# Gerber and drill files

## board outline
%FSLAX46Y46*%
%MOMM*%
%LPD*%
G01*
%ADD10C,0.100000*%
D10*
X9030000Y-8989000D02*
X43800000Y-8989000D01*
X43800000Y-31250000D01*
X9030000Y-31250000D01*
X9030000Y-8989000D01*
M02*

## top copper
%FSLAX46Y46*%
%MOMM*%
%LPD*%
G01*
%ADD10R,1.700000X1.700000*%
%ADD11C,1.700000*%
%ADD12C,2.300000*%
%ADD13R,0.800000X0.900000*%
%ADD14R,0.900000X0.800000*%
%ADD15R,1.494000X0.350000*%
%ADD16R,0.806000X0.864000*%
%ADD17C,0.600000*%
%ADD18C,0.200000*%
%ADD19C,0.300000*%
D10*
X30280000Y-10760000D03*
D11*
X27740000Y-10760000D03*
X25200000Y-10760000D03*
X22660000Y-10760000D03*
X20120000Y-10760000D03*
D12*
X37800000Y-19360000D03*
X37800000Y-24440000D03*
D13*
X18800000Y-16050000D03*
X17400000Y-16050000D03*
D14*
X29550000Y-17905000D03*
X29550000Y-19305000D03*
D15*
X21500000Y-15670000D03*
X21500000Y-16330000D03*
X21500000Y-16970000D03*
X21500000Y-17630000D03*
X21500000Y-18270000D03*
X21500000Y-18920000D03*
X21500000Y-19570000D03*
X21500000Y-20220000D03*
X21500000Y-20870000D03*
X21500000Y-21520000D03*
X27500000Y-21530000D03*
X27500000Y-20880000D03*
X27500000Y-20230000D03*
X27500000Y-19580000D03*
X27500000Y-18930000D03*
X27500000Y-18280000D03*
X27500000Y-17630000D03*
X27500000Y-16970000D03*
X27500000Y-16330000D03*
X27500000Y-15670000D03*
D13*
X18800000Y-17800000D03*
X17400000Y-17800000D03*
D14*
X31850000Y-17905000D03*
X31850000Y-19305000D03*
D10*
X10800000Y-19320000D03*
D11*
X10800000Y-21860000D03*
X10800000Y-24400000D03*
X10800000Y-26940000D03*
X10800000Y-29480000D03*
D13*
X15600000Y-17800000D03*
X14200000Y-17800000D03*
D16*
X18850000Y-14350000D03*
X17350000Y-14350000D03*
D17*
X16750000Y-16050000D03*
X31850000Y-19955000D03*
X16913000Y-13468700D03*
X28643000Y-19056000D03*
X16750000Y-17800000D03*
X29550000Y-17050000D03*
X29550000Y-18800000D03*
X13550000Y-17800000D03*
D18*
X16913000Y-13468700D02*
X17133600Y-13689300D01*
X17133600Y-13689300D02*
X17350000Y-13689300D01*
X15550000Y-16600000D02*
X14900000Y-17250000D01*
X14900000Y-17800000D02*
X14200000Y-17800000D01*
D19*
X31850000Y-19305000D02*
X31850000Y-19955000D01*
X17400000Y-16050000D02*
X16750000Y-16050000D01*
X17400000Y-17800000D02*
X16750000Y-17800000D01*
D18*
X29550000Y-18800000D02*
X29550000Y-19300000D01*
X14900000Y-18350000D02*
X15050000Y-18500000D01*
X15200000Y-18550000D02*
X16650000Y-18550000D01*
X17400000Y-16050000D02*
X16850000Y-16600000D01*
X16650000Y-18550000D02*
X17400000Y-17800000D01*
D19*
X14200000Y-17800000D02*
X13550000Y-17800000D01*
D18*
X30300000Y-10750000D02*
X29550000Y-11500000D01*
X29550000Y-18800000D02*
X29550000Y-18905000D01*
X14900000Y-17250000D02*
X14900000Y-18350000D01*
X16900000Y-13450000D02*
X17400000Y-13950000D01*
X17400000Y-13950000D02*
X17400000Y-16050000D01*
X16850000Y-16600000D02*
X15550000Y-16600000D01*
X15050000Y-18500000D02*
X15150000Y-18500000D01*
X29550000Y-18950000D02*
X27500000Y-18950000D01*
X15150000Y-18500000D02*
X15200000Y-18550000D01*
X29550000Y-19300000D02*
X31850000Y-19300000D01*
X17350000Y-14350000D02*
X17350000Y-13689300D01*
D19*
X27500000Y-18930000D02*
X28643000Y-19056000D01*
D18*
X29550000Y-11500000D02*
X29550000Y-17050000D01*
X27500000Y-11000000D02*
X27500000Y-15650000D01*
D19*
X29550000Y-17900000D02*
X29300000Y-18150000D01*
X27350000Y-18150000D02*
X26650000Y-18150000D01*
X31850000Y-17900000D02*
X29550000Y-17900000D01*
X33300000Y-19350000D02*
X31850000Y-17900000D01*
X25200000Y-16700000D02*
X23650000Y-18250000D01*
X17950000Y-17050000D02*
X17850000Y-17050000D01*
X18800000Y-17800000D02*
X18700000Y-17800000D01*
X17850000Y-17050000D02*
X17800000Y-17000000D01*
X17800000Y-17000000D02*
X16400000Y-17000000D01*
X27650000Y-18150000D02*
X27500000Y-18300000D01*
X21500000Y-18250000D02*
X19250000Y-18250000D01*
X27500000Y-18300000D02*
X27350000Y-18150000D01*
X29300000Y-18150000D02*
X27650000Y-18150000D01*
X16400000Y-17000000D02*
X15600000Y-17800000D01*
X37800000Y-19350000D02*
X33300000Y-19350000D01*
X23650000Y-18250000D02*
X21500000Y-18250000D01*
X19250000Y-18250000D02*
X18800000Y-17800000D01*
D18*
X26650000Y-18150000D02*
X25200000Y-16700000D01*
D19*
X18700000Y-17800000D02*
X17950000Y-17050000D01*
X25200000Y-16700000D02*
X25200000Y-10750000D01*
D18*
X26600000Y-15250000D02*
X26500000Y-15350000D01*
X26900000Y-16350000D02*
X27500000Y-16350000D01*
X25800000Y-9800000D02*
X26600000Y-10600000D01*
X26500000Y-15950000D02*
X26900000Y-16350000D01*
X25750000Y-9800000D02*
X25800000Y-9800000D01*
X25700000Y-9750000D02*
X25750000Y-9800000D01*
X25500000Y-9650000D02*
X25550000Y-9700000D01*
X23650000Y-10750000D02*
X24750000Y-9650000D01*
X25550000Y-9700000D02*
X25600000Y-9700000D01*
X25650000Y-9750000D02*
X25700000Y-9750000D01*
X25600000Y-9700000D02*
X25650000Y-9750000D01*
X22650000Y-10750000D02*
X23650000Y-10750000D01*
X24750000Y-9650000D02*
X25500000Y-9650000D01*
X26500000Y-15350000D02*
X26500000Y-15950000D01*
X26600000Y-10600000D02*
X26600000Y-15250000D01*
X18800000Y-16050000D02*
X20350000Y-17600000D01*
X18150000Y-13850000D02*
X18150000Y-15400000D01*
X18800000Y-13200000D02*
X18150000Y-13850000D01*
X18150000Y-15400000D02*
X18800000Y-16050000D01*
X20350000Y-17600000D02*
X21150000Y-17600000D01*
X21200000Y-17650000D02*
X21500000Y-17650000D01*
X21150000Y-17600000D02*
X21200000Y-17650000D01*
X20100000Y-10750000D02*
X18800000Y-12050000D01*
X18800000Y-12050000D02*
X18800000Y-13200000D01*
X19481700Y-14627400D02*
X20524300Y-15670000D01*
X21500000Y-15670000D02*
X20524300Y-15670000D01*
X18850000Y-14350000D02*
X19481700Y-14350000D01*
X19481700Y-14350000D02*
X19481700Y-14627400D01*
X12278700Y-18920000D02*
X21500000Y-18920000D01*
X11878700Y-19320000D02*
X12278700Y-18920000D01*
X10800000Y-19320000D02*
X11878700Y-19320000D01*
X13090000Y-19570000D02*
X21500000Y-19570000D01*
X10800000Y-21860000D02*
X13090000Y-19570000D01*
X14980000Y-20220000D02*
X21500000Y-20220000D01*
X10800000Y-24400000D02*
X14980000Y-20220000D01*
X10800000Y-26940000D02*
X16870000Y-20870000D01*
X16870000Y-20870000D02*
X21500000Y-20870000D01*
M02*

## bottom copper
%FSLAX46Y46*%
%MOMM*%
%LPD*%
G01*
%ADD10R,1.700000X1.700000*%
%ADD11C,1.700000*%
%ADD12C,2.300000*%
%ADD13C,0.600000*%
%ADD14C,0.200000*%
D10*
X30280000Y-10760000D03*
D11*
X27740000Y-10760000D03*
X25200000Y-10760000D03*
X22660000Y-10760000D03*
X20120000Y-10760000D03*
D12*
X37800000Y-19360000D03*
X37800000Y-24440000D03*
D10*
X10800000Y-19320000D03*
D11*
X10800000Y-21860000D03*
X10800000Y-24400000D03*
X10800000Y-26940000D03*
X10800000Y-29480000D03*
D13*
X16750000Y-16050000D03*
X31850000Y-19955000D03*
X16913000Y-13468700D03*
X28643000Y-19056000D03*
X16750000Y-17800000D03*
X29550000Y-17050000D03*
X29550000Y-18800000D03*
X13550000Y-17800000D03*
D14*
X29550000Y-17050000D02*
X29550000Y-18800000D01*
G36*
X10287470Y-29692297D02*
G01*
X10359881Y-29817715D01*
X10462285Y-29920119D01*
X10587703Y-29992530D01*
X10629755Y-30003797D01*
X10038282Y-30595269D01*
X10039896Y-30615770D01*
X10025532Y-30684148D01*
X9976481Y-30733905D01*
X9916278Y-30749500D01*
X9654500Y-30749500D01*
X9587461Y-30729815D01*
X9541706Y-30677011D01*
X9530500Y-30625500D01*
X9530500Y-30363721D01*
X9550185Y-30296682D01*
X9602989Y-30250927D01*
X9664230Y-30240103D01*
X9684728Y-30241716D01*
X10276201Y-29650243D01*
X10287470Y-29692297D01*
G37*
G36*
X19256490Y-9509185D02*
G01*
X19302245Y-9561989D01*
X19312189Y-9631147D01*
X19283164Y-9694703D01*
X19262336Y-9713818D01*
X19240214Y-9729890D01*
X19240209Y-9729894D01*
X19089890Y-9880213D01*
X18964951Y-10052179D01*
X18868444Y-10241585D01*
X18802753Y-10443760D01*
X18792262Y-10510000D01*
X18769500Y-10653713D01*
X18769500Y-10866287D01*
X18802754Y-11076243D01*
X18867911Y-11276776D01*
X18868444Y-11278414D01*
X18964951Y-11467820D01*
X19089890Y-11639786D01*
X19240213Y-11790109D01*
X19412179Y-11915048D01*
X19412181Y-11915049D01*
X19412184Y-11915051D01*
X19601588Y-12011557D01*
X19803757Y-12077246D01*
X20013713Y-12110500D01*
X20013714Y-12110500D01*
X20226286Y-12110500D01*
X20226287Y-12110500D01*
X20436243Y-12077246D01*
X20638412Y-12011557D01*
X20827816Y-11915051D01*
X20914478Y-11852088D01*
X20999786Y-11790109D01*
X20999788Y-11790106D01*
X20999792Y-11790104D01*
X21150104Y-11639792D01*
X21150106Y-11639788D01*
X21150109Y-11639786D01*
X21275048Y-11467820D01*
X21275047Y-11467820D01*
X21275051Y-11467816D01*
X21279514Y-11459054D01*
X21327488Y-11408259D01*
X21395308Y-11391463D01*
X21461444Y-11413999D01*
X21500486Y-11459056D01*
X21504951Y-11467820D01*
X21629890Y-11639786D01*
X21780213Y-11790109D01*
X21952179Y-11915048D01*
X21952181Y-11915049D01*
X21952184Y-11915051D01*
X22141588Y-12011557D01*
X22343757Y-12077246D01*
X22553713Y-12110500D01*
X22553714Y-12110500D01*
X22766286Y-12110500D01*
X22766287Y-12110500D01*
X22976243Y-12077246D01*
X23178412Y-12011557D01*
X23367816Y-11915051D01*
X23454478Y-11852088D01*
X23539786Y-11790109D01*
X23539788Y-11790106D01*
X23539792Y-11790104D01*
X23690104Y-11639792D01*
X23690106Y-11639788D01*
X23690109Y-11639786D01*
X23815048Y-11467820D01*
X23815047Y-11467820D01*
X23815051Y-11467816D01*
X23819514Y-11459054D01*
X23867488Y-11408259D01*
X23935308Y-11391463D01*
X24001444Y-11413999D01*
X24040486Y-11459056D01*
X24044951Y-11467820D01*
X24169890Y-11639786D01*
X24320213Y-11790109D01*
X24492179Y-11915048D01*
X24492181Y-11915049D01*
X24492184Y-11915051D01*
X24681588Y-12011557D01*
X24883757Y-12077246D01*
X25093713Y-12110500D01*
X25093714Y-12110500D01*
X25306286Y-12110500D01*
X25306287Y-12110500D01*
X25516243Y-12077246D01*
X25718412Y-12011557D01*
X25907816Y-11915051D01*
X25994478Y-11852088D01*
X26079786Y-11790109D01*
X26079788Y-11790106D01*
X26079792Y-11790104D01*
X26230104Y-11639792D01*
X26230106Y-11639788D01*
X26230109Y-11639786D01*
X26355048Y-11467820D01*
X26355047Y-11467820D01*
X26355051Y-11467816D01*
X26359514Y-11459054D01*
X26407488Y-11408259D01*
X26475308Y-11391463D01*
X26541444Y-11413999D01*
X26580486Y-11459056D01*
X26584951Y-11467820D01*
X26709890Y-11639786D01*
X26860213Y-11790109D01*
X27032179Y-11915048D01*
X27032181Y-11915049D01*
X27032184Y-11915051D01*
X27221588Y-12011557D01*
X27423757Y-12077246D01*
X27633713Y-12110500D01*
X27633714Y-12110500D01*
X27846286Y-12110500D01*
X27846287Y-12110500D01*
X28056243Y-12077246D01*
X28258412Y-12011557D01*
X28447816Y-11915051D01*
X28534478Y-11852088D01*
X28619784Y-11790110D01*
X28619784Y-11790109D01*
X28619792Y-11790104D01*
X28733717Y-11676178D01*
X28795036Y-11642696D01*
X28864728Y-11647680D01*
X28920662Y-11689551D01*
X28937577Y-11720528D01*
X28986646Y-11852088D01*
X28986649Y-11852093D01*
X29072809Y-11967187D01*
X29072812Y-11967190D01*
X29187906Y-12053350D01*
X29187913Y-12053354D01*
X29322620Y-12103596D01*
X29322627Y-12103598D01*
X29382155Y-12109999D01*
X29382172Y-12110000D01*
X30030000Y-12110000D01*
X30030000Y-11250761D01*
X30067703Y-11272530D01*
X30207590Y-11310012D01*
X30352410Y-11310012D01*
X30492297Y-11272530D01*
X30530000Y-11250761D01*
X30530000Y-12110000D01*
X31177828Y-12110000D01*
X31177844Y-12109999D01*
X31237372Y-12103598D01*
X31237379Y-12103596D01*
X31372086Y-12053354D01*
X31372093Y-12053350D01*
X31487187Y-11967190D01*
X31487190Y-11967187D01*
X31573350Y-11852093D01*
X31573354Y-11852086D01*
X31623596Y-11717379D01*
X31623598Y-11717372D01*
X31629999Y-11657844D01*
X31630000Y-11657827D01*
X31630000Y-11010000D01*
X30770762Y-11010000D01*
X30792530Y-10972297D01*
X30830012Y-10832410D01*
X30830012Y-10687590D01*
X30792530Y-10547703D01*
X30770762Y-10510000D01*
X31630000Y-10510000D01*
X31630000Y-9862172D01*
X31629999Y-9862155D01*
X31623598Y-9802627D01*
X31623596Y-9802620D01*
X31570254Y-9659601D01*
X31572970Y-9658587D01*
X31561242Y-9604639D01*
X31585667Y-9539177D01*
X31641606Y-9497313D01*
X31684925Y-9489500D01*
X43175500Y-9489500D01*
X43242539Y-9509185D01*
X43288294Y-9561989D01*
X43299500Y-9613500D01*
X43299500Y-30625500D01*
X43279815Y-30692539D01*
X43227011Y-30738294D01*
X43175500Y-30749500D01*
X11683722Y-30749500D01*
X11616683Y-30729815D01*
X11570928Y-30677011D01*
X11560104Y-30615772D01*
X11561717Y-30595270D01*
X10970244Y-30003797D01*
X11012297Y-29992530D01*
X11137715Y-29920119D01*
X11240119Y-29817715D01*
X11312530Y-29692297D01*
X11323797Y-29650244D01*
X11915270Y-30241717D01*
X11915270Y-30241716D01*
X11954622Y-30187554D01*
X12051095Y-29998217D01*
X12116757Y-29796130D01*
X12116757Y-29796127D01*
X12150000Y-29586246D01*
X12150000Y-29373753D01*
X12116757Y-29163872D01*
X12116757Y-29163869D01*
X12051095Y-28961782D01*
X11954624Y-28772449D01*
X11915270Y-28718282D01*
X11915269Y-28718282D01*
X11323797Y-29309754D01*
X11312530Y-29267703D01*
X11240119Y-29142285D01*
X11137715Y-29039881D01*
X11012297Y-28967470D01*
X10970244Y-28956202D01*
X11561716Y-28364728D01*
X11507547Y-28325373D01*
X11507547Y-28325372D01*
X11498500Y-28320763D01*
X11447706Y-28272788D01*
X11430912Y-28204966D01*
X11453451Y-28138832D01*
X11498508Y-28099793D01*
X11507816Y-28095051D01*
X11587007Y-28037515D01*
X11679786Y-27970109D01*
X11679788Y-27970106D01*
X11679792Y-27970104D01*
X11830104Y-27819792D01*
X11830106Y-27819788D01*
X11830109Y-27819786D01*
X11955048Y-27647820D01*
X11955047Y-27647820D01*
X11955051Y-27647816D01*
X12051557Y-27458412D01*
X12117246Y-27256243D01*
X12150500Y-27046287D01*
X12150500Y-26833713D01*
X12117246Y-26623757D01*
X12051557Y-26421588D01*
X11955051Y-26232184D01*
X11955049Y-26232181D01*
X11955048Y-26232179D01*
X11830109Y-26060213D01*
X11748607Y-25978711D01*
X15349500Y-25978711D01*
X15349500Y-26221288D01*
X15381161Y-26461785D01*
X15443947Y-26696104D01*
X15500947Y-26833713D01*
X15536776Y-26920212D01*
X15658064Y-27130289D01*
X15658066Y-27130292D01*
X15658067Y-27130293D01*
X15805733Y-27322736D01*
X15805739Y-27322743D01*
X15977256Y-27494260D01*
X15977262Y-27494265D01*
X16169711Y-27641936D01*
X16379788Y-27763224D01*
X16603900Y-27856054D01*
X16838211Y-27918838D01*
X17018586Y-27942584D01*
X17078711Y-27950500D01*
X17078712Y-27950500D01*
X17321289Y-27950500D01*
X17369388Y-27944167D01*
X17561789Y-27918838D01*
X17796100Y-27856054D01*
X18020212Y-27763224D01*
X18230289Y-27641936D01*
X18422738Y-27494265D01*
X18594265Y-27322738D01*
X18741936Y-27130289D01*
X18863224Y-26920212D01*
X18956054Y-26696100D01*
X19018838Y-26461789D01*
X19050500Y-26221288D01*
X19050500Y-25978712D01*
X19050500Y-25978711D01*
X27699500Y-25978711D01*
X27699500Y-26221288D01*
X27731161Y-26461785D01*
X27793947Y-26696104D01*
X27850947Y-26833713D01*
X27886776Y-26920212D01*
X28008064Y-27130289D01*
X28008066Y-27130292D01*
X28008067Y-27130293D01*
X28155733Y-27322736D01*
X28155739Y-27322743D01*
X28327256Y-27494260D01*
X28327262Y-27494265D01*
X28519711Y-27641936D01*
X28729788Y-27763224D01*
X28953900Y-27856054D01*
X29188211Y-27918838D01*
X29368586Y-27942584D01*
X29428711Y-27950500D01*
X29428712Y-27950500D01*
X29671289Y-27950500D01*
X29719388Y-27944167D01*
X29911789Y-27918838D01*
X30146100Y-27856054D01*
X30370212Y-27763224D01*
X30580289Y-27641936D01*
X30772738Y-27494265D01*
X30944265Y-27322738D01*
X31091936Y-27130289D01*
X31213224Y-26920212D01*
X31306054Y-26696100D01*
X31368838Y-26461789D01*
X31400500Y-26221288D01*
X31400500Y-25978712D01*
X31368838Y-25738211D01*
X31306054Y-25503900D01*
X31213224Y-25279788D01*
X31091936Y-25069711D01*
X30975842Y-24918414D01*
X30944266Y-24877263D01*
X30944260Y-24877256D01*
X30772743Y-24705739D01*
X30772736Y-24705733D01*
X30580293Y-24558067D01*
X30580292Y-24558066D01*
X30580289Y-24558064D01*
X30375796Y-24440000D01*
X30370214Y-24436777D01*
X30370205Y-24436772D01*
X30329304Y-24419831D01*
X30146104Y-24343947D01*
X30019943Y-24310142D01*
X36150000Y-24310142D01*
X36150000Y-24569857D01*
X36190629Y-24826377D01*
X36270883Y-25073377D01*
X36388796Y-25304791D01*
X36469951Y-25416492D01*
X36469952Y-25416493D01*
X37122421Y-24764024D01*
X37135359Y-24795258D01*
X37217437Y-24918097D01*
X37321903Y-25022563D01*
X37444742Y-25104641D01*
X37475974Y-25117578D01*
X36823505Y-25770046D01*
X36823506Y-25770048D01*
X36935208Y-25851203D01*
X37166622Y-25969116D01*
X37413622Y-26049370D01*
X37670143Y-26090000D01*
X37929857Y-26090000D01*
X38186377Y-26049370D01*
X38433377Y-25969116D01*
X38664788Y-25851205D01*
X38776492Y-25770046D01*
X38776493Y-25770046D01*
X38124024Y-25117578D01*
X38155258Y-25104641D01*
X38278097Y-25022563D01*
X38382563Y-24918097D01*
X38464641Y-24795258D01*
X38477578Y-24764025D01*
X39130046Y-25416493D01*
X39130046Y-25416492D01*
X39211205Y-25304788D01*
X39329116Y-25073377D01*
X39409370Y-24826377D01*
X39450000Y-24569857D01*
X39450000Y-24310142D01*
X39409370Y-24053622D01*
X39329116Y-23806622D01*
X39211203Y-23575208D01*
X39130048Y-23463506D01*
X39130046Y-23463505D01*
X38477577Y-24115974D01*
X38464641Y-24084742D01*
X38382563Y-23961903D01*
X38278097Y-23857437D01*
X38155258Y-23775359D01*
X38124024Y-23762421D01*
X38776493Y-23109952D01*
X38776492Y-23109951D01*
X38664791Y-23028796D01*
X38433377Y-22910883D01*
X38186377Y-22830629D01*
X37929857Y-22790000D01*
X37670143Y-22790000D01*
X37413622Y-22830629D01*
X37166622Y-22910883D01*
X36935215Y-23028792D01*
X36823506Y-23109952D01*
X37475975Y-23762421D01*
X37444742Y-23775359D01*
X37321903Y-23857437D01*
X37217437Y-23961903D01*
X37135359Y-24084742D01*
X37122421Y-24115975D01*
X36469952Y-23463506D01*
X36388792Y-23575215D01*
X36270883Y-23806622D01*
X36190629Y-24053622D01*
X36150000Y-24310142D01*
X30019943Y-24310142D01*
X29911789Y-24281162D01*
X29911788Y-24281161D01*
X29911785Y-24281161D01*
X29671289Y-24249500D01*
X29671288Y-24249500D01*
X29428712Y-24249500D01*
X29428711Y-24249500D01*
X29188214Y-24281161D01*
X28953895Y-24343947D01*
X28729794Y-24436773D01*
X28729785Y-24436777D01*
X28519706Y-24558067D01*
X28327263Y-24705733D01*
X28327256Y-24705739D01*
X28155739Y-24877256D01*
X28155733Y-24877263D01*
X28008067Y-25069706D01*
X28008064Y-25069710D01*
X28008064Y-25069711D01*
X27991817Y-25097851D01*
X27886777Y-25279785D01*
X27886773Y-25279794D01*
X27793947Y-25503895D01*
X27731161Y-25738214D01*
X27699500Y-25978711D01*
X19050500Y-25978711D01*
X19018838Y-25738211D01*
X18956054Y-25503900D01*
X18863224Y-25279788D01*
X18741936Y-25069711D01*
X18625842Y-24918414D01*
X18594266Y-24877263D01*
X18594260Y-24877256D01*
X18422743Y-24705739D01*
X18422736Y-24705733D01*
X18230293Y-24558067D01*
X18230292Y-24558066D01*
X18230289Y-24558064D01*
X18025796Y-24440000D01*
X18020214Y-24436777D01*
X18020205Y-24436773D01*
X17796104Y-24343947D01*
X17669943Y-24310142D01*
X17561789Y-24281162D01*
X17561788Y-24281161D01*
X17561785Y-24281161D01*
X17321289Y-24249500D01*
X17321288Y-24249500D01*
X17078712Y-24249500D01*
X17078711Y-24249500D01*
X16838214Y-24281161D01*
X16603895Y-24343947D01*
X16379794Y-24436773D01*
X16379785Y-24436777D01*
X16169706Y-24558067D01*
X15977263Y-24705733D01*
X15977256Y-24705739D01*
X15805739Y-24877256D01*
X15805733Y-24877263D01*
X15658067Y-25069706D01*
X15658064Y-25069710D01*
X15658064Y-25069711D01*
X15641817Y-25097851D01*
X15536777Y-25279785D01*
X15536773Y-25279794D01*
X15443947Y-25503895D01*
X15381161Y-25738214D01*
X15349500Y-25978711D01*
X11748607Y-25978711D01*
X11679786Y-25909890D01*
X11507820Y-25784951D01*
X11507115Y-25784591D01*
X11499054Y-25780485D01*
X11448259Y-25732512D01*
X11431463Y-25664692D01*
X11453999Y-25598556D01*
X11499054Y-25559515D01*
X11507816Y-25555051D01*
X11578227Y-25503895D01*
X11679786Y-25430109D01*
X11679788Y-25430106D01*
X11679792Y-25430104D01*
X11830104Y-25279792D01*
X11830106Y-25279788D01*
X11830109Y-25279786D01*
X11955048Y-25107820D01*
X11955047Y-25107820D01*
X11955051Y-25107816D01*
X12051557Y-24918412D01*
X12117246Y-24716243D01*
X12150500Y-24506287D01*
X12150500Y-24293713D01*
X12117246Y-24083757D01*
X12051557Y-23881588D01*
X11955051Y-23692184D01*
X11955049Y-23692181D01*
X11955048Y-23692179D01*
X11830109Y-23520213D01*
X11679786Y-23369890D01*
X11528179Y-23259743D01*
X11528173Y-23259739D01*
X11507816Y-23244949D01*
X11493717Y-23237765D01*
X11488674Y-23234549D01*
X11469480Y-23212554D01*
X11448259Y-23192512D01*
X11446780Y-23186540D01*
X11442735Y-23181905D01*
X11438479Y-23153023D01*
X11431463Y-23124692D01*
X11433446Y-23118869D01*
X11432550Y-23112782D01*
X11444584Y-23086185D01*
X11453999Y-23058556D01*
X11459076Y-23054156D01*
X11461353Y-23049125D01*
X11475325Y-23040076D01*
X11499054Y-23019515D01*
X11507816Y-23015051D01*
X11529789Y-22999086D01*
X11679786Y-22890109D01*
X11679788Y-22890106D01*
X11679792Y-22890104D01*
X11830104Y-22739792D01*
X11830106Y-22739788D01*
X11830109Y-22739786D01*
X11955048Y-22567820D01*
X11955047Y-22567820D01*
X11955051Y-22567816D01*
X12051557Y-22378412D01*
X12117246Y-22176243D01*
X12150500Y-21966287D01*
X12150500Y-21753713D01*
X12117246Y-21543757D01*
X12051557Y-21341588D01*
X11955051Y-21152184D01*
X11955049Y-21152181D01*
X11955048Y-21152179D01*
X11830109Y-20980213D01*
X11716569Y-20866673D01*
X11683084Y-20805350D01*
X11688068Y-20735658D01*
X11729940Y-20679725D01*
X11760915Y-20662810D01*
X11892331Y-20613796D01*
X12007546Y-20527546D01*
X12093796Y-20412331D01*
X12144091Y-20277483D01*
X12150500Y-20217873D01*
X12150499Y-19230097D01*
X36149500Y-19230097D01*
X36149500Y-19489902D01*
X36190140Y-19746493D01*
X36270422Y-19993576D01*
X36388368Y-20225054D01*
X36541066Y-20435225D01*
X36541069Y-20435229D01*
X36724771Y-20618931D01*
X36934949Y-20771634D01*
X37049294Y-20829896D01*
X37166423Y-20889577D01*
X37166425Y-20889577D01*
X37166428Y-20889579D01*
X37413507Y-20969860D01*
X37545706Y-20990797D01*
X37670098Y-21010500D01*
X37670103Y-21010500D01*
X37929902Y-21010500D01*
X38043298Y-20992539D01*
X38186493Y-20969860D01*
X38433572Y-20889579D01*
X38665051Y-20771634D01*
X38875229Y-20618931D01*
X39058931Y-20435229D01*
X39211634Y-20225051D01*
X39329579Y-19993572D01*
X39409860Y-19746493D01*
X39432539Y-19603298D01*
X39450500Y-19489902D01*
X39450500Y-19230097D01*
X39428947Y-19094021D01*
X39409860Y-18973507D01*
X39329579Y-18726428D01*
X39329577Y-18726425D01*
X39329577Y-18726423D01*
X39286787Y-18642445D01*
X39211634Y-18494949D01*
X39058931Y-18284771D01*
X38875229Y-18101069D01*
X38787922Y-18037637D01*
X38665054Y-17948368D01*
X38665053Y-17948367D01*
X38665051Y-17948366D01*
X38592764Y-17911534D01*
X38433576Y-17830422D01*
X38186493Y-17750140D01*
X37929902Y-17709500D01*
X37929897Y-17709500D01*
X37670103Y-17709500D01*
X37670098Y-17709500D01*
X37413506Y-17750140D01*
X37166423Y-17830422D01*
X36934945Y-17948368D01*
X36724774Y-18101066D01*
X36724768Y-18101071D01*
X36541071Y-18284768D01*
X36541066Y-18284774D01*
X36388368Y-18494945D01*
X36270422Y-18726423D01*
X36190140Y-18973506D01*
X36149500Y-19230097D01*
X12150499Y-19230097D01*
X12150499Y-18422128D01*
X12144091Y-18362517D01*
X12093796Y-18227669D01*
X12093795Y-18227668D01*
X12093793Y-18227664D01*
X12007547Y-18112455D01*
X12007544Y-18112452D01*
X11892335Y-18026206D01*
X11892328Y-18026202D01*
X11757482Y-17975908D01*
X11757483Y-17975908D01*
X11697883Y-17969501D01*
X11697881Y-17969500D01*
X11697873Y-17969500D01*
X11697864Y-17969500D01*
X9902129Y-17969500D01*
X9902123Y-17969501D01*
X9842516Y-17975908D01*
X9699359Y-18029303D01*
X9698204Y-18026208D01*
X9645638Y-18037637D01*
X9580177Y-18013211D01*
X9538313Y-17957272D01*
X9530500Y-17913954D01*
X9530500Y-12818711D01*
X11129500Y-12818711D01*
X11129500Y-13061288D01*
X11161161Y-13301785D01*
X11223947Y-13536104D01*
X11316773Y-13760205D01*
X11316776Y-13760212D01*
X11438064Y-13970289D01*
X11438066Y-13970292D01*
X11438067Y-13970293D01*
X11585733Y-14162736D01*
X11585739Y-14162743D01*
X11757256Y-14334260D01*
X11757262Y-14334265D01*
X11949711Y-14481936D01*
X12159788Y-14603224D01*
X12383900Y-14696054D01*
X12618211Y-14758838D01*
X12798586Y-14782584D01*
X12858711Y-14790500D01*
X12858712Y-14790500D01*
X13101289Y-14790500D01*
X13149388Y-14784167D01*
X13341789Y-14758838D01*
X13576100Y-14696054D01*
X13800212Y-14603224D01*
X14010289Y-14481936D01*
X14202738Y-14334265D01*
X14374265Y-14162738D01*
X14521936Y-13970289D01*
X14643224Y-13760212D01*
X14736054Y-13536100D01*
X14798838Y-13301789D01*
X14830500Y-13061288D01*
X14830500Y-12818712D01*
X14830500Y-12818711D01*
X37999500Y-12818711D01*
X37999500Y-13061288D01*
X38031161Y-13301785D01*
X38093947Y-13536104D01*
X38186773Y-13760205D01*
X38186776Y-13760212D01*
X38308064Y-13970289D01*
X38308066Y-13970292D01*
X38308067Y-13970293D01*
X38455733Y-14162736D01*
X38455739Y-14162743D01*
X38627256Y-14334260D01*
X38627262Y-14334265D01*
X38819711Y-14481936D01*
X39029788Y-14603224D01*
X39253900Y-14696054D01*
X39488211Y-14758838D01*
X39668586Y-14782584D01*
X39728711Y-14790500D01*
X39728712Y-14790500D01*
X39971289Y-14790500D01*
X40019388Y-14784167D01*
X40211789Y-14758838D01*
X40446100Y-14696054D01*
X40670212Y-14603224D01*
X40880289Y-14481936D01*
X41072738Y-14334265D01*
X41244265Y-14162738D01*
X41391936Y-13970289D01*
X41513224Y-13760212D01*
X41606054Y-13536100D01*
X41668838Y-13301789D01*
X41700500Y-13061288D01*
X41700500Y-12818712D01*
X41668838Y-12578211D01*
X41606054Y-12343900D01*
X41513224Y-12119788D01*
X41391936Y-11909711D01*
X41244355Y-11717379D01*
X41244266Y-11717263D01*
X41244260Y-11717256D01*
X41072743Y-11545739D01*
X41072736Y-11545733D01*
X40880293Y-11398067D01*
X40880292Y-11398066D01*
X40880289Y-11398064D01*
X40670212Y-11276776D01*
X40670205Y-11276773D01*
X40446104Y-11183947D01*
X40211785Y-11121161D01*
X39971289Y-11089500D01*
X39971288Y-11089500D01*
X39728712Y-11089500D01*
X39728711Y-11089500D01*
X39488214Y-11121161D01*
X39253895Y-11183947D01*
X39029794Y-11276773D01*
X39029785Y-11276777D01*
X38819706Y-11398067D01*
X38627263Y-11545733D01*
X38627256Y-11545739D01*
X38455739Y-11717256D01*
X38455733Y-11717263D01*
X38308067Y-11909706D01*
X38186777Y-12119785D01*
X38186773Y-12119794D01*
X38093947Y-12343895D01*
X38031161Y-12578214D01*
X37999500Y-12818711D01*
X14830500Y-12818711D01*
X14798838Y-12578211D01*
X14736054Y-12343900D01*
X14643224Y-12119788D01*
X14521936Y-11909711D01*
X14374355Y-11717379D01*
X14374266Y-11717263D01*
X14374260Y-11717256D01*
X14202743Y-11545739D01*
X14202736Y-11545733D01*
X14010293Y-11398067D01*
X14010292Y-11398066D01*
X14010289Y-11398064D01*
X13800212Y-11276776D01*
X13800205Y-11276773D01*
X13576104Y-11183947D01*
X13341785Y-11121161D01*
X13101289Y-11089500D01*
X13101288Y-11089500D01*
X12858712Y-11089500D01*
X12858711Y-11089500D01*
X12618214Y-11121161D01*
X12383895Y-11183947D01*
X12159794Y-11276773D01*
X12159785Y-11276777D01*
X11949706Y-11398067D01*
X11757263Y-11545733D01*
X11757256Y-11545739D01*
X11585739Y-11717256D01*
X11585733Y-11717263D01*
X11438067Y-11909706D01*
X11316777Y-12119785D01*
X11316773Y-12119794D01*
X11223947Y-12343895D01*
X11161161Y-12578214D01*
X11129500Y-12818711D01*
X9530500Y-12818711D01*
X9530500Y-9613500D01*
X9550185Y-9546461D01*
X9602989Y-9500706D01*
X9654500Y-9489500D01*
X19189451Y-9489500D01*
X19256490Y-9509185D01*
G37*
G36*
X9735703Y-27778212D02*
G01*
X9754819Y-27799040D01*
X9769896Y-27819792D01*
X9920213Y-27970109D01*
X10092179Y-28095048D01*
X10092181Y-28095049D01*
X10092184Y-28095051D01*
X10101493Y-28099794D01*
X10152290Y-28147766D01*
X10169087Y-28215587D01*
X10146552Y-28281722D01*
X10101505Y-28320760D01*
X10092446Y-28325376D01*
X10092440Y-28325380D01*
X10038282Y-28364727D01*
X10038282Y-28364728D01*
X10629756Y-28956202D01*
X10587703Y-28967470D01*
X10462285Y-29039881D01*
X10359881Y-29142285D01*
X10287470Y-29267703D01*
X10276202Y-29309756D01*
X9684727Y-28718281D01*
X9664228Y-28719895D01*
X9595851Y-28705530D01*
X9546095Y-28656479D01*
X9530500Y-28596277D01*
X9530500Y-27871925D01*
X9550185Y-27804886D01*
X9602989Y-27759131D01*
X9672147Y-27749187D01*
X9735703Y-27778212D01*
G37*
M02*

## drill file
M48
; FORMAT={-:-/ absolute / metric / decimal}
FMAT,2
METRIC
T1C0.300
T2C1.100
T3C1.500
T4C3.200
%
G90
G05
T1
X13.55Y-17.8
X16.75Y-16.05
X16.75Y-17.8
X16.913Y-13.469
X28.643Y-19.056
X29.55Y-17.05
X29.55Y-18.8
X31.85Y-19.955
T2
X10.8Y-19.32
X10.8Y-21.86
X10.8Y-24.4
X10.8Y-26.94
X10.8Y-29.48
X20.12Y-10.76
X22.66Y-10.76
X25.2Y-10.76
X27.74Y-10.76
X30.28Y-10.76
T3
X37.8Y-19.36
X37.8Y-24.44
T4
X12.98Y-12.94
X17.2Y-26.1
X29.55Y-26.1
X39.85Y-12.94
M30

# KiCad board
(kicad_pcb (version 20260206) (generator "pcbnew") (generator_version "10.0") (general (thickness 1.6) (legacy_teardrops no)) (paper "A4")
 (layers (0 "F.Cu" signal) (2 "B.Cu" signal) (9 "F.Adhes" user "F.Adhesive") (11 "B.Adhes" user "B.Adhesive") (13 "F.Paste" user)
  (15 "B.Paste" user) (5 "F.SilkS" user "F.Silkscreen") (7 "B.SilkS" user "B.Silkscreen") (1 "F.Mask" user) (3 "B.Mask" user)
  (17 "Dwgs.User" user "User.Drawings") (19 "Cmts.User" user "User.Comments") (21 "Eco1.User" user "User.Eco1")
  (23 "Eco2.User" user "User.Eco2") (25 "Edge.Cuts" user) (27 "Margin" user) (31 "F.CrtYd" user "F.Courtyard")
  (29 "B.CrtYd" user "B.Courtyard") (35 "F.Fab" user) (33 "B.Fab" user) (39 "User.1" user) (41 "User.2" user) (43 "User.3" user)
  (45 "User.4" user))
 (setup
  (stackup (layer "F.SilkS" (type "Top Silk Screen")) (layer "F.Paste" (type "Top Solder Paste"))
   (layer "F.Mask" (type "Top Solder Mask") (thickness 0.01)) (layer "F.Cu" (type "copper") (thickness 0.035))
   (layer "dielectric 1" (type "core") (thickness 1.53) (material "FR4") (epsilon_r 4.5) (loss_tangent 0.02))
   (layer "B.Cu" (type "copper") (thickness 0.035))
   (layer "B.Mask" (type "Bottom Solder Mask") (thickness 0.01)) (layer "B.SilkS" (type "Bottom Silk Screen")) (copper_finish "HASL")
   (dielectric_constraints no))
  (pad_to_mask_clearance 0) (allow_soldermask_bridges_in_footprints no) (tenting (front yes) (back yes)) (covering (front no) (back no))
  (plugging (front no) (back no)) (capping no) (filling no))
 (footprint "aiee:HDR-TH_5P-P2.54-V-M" (layer "F.Cu") (at 25.2 10.76 180)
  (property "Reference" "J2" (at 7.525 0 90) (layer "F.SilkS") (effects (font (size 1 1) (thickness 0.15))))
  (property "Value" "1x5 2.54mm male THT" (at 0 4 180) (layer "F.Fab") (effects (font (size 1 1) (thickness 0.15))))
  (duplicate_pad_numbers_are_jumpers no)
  (pad "1" thru_hole rect (at -5.08 0 180) (size 1.7 1.7) (drill 1.100024) (layers "*.Cu" "*.Mask") (remove_unused_layers no) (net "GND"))
  (pad "2" thru_hole circle (at -2.54 0 180) (size 1.7 1.7) (drill 1.100024) (layers "*.Cu" "*.Mask") (remove_unused_layers no)
   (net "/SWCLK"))
  (pad "3" thru_hole circle (at 0 0 180) (size 1.7 1.7) (drill 1.100024) (layers "*.Cu" "*.Mask") (remove_unused_layers no) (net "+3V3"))
  (pad "4" thru_hole circle (at 2.54 0 180) (size 1.7 1.7) (drill 1.100024) (layers "*.Cu" "*.Mask") (remove_unused_layers no)
   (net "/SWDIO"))
  (pad "5" thru_hole circle (at 5.08 0 180) (size 1.7 1.7) (drill 1.100024) (layers "*.Cu" "*.Mask") (remove_unused_layers no) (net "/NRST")))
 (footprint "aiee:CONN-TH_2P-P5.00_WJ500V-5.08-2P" (layer "F.Cu") (at 37.8 21.9 -90)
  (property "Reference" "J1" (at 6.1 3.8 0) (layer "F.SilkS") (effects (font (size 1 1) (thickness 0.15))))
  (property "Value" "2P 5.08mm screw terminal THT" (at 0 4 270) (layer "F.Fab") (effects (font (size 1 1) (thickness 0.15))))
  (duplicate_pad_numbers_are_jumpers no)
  (pad "1" thru_hole circle (at -2.54 0 90) (size 2.3 2.3) (drill 1.5) (layers "*.Cu" "*.Mask") (remove_unused_layers no) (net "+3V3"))
  (pad "2" thru_hole circle (at 2.54 0 90) (size 2.3 2.3) (drill 1.5) (layers "*.Cu" "*.Mask") (remove_unused_layers no) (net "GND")))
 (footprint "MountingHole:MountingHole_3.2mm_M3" (layer "F.Cu") (at 29.55 26.1)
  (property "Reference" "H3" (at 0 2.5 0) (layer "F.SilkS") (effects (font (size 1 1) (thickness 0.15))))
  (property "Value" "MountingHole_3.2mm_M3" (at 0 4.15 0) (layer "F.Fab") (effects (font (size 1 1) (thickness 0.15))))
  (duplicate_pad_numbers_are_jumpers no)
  (pad "" np_thru_hole circle (at 0 0) (size 3.2 3.2) (drill 3.2) (layers "*.Cu" "*.Mask")))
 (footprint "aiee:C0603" (layer "F.Cu") (at 18.1 16.05 180)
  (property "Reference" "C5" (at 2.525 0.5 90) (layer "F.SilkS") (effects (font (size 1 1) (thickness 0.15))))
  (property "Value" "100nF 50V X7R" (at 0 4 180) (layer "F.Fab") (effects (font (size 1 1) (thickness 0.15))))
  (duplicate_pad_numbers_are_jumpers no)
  (pad "1" smd rect (at -0.7 0 180) (size 0.8 0.9) (layers "F.Cu" "F.Mask" "F.Paste") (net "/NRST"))
  (pad "2" smd rect (at 0.7 0 180) (size 0.8 0.9) (layers "F.Cu" "F.Mask" "F.Paste") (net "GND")))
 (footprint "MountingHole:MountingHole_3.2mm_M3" (layer "F.Cu") (at 17.2 26.1)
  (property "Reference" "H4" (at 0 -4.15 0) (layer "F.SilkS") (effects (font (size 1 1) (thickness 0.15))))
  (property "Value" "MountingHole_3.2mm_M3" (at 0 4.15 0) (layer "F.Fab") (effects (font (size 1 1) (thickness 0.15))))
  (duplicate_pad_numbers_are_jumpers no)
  (pad "" np_thru_hole circle (at 0 0) (size 3.2 3.2) (drill 3.2) (layers "*.Cu" "*.Mask")))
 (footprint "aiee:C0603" (layer "F.Cu") (at 29.55 18.605 -90)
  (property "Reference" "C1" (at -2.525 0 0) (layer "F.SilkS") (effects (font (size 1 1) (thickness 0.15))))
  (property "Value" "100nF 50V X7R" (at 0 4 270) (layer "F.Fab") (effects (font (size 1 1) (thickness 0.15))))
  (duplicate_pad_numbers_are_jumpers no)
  (pad "1" smd rect (at -0.7 0 270) (size 0.8 0.9) (layers "F.Cu" "F.Mask" "F.Paste") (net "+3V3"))
  (pad "2" smd rect (at 0.7 0 270) (size 0.8 0.9) (layers "F.Cu" "F.Mask" "F.Paste") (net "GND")))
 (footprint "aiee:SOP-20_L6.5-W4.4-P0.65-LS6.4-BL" (layer "F.Cu") (at 24.5 18.6 -90)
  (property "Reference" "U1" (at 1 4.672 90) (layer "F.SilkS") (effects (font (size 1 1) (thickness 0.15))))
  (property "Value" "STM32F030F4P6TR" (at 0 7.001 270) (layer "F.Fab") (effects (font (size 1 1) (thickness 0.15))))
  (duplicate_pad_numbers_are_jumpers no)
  (pad "1" smd rect (at -2.93 3 270) (size 0.35 1.494) (layers "F.Cu" "F.Mask" "F.Paste") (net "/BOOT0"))
  (pad "2" smd rect (at -2.27 3 270) (size 0.35 1.494) (layers "F.Cu" "F.Mask" "F.Paste") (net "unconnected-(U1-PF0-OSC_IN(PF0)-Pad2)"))
  (pad "3" smd rect (at -1.63 3 270) (size 0.35 1.494) (layers "F.Cu" "F.Mask" "F.Paste") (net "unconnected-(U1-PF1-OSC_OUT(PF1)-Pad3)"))
  (pad "4" smd rect (at -0.97 3 270) (size 0.35 1.494) (layers "F.Cu" "F.Mask" "F.Paste") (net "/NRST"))
  (pad "5" smd rect (at -0.33 3 270) (size 0.35 1.494) (layers "F.Cu" "F.Mask" "F.Paste") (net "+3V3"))
  (pad "6" smd rect (at 0.32 3 270) (size 0.35 1.494) (layers "F.Cu" "F.Mask" "F.Paste") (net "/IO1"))
  (pad "7" smd rect (at 0.97 3 270) (size 0.35 1.494) (layers "F.Cu" "F.Mask" "F.Paste") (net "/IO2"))
  (pad "8" smd rect (at 1.62 3 270) (size 0.35 1.494) (layers "F.Cu" "F.Mask" "F.Paste") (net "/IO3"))
  (pad "9" smd rect (at 2.27 3 270) (size 0.35 1.494) (layers "F.Cu" "F.Mask" "F.Paste") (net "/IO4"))
  (pad "10" smd rect (at 2.92 3 270) (size 0.35 1.494) (layers "F.Cu" "F.Mask" "F.Paste") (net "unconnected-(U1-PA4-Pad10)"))
  (pad "11" smd rect (at 2.93 -3 270) (size 0.35 1.494) (layers "F.Cu" "F.Mask" "F.Paste") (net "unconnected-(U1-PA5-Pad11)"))
  (pad "12" smd rect (at 2.28 -3 270) (size 0.35 1.494) (layers "F.Cu" "F.Mask" "F.Paste") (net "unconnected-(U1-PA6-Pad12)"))
  (pad "13" smd rect (at 1.63 -3 270) (size 0.35 1.494) (layers "F.Cu" "F.Mask" "F.Paste") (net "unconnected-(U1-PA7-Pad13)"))
  (pad "14" smd rect (at 0.98 -3 270) (size 0.35 1.494) (layers "F.Cu" "F.Mask" "F.Paste") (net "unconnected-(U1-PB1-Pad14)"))
  (pad "15" smd rect (at 0.33 -3 270) (size 0.35 1.494) (layers "F.Cu" "F.Mask" "F.Paste") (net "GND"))
  (pad "16" smd rect (at -0.32 -3 270) (size 0.35 1.494) (layers "F.Cu" "F.Mask" "F.Paste") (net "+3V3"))
  (pad "17" smd rect (at -0.97 -3 270) (size 0.35 1.494) (layers "F.Cu" "F.Mask" "F.Paste") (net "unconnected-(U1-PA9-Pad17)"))
  (pad "18" smd rect (at -1.63 -3 270) (size 0.35 1.494) (layers "F.Cu" "F.Mask" "F.Paste") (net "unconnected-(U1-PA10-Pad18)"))
  (pad "19" smd rect (at -2.27 -3 270) (size 0.35 1.494) (layers "F.Cu" "F.Mask" "F.Paste") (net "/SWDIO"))
  (pad "20" smd rect (at -2.93 -3 270) (size 0.35 1.494) (layers "F.Cu" "F.Mask" "F.Paste") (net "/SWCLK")))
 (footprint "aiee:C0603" (layer "F.Cu") (at 18.1 17.8 180)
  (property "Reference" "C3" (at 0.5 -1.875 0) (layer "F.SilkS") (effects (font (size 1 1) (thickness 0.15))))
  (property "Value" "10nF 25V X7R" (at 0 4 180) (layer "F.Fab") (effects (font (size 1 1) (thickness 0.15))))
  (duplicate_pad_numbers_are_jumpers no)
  (pad "1" smd rect (at -0.7 0 180) (size 0.8 0.9) (layers "F.Cu" "F.Mask" "F.Paste") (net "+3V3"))
  (pad "2" smd rect (at 0.7 0 180) (size 0.8 0.9) (layers "F.Cu" "F.Mask" "F.Paste") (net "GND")))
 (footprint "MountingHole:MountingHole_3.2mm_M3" (layer "F.Cu") (at 12.98 12.94)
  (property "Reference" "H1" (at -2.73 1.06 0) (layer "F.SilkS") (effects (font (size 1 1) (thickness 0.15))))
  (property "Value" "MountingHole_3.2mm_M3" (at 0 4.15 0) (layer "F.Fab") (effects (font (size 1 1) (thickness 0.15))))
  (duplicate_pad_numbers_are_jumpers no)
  (pad "" np_thru_hole circle (at 0 0) (size 3.2 3.2) (drill 3.2) (layers "*.Cu" "*.Mask")))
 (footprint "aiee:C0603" (layer "F.Cu") (at 31.85 18.605 -90)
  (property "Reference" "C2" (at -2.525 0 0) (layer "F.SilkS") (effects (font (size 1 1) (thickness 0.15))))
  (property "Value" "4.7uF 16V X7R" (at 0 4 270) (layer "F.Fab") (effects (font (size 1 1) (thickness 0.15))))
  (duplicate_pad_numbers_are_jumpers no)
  (pad "1" smd rect (at -0.7 0 270) (size 0.8 0.9) (layers "F.Cu" "F.Mask" "F.Paste") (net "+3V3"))
  (pad "2" smd rect (at 0.7 0 270) (size 0.8 0.9) (layers "F.Cu" "F.Mask" "F.Paste") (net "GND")))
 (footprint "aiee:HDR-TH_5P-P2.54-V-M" (layer "F.Cu") (at 10.8 24.4 -90)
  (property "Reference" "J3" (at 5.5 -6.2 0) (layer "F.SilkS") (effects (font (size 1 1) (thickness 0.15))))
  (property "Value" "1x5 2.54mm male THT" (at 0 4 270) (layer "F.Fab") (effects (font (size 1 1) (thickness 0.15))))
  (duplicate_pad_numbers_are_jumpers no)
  (pad "1" thru_hole rect (at -5.08 0 270) (size 1.7 1.7) (drill 1.100024) (layers "*.Cu" "*.Mask") (remove_unused_layers no) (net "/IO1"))
  (pad "2" thru_hole circle (at -2.54 0 270) (size 1.7 1.7) (drill 1.100024) (layers "*.Cu" "*.Mask") (remove_unused_layers no) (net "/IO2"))
  (pad "3" thru_hole circle (at 0 0 270) (size 1.7 1.7) (drill 1.100024) (layers "*.Cu" "*.Mask") (remove_unused_layers no) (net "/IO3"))
  (pad "4" thru_hole circle (at 2.54 0 270) (size 1.7 1.7) (drill 1.100024) (layers "*.Cu" "*.Mask") (remove_unused_layers no) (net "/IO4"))
  (pad "5" thru_hole circle (at 5.08 0 270) (size 1.7 1.7) (drill 1.100024) (layers "*.Cu" "*.Mask") (remove_unused_layers no) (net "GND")))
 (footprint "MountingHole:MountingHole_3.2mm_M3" (layer "F.Cu") (at 39.85 12.94)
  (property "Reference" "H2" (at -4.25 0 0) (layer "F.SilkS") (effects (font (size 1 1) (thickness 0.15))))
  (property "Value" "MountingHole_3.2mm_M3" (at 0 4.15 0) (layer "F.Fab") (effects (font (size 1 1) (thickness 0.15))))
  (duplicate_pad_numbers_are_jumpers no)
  (pad "" np_thru_hole circle (at 0 0) (size 3.2 3.2) (drill 3.2) (layers "*.Cu" "*.Mask")))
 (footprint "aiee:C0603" (layer "F.Cu") (at 14.9 17.8 180)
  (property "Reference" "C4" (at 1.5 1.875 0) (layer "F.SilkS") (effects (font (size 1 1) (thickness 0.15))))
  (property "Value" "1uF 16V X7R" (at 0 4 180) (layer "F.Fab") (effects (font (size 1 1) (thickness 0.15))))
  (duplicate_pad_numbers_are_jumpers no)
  (pad "1" smd rect (at -0.7 0 180) (size 0.8 0.9) (layers "F.Cu" "F.Mask" "F.Paste") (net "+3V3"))
  (pad "2" smd rect (at 0.7 0 180) (size 0.8 0.9) (layers "F.Cu" "F.Mask" "F.Paste") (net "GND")))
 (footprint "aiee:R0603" (layer "F.Cu") (at 18.1 14.35 180)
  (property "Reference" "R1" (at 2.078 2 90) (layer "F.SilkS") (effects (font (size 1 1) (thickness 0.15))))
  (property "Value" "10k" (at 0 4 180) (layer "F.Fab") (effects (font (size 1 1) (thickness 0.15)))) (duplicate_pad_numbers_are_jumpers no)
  (pad "1" smd rect (at -0.75 0 180) (size 0.806 0.864) (layers "F.Cu" "F.Mask" "F.Paste") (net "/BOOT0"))
  (pad "2" smd rect (at 0.75 0 180) (size 0.806 0.864) (layers "F.Cu" "F.Mask" "F.Paste") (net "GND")))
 (gr_rect (start 9.03 8.989) (end 43.8 31.25) (stroke (width 0.1) (type default)) (fill no) (layer "Edge.Cuts"))
 (segment (start 16.913 13.4687) (end 17.1336 13.6893) (width 0.2) (layer "F.Cu") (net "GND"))
 (segment (start 17.1336 13.6893) (end 17.35 13.6893) (width 0.2) (layer "F.Cu") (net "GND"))
 (segment (start 15.55 16.6) (end 14.9 17.25) (width 0.2) (layer "F.Cu") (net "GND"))
 (segment (start 14.9 17.8) (end 14.2 17.8) (width 0.2) (layer "F.Cu") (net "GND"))
 (segment (start 31.85 19.305) (end 31.85 19.955) (width 0.3) (layer "F.Cu") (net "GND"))
 (segment (start 17.4 16.05) (end 16.75 16.05) (width 0.3) (layer "F.Cu") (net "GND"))
 (segment (start 17.4 17.8) (end 16.75 17.8) (width 0.3) (layer "F.Cu") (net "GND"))
 (segment (start 29.55 18.8) (end 29.55 19.3) (width 0.2) (layer "F.Cu") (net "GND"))
 (segment (start 14.9 18.35) (end 15.05 18.5) (width 0.2) (layer "F.Cu") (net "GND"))
 (segment (start 15.2 18.55) (end 16.65 18.55) (width 0.2) (layer "F.Cu") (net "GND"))
 (segment (start 17.4 16.05) (end 16.85 16.6) (width 0.2) (layer "F.Cu") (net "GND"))
 (segment (start 16.65 18.55) (end 17.4 17.8) (width 0.2) (layer "F.Cu") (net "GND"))
 (segment (start 14.2 17.8) (end 13.55 17.8) (width 0.3) (layer "F.Cu") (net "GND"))
 (segment (start 30.3 10.75) (end 29.55 11.5) (width 0.2) (layer "F.Cu") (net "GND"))
 (segment (start 29.55 18.8) (end 29.55 18.905) (width 0.2) (layer "F.Cu") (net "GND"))
 (segment (start 14.9 17.25) (end 14.9 18.35) (width 0.2) (layer "F.Cu") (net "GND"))
 (segment (start 16.9 13.45) (end 17.4 13.95) (width 0.2) (layer "F.Cu") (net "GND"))
 (segment (start 17.4 13.95) (end 17.4 16.05) (width 0.2) (layer "F.Cu") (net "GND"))
 (segment (start 16.85 16.6) (end 15.55 16.6) (width 0.2) (layer "F.Cu") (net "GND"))
 (segment (start 15.05 18.5) (end 15.15 18.5) (width 0.2) (layer "F.Cu") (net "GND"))
 (segment (start 29.55 18.95) (end 27.5 18.95) (width 0.2) (layer "F.Cu") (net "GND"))
 (segment (start 15.15 18.5) (end 15.2 18.55) (width 0.2) (layer "F.Cu") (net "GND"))
 (segment (start 29.55 19.3) (end 31.85 19.3) (width 0.2) (layer "F.Cu") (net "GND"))
 (segment (start 17.35 14.35) (end 17.35 13.6893) (width 0.2) (layer "F.Cu") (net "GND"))
 (segment (start 27.5 18.93) (end 28.643 19.056) (width 0.3) (layer "F.Cu") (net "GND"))
 (segment (start 29.55 11.5) (end 29.55 17.05) (width 0.2) (layer "F.Cu") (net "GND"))
 (via (at 16.75 16.05) (size 0.6) (drill 0.3) (layers "F.Cu" "B.Cu") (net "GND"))
 (via (at 31.85 19.955) (size 0.6) (drill 0.3) (layers "F.Cu" "B.Cu") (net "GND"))
 (via (at 16.913 13.4687) (size 0.6) (drill 0.3) (layers "F.Cu" "B.Cu") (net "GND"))
 (via (at 28.643 19.056) (size 0.6) (drill 0.3) (layers "F.Cu" "B.Cu") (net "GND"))
 (via (at 16.75 17.8) (size 0.6) (drill 0.3) (layers "F.Cu" "B.Cu") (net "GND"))
 (via (at 29.55 17.05) (size 0.6) (drill 0.3) (layers "F.Cu" "B.Cu") (tenting (front yes) (back yes)) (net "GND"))
 (via (at 29.55 18.8) (size 0.6) (drill 0.3) (layers "F.Cu" "B.Cu") (tenting (front yes) (back yes)) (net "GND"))
 (via (at 13.55 17.8) (size 0.6) (drill 0.3) (layers "F.Cu" "B.Cu") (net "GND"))
 (segment (start 29.55 17.05) (end 29.55 18.8) (width 0.2) (layer "B.Cu") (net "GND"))
 (segment (start 27.5 11) (end 27.5 15.65) (width 0.2) (layer "F.Cu") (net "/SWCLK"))
 (segment (start 29.55 17.9) (end 29.3 18.15) (width 0.3) (layer "F.Cu") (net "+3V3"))
 (segment (start 27.35 18.15) (end 26.65 18.15) (width 0.3) (layer "F.Cu") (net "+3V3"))
 (segment (start 31.85 17.9) (end 29.55 17.9) (width 0.3) (layer "F.Cu") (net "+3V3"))
 (segment (start 33.3 19.35) (end 31.85 17.9) (width 0.3) (layer "F.Cu") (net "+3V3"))
 (segment (start 25.2 16.7) (end 23.65 18.25) (width 0.3) (layer "F.Cu") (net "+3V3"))
 (segment (start 17.95 17.05) (end 17.85 17.05) (width 0.3) (layer "F.Cu") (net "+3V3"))
 (segment (start 18.8 17.8) (end 18.7 17.8) (width 0.3) (layer "F.Cu") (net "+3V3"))
 (segment (start 17.85 17.05) (end 17.8 17) (width 0.3) (layer "F.Cu") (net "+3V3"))
 (segment (start 17.8 17) (end 16.4 17) (width 0.3) (layer "F.Cu") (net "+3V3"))
 (segment (start 27.65 18.15) (end 27.5 18.3) (width 0.3) (layer "F.Cu") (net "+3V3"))
 (segment (start 21.5 18.25) (end 19.25 18.25) (width 0.3) (layer "F.Cu") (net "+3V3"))
 (segment (start 27.5 18.3) (end 27.35 18.15) (width 0.3) (layer "F.Cu") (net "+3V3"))
 (segment (start 29.3 18.15) (end 27.65 18.15) (width 0.3) (layer "F.Cu") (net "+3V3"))
 (segment (start 16.4 17) (end 15.6 17.8) (width 0.3) (layer "F.Cu") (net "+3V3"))
 (segment (start 37.8 19.35) (end 33.3 19.35) (width 0.3) (layer "F.Cu") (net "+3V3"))
 (segment (start 23.65 18.25) (end 21.5 18.25) (width 0.3) (layer "F.Cu") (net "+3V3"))
 (segment (start 19.25 18.25) (end 18.8 17.8) (width 0.3) (layer "F.Cu") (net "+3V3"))
 (segment (start 26.65 18.15) (end 25.2 16.7) (width 0.2) (layer "F.Cu") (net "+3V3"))
 (segment (start 18.7 17.8) (end 17.95 17.05) (width 0.3) (layer "F.Cu") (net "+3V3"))
 (segment (start 25.2 16.7) (end 25.2 10.75) (width 0.3) (layer "F.Cu") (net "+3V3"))
 (segment (start 26.6 15.25) (end 26.5 15.35) (width 0.2) (layer "F.Cu") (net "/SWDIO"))
 (segment (start 26.9 16.35) (end 27.5 16.35) (width 0.2) (layer "F.Cu") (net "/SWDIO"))
 (segment (start 25.8 9.8) (end 26.6 10.6) (width 0.2) (layer "F.Cu") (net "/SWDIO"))
 (segment (start 26.5 15.95) (end 26.9 16.35) (width 0.2) (layer "F.Cu") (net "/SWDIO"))
 (segment (start 25.75 9.8) (end 25.8 9.8) (width 0.2) (layer "F.Cu") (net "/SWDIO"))
 (segment (start 25.7 9.75) (end 25.75 9.8) (width 0.2) (layer "F.Cu") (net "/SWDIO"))
 (segment (start 25.5 9.65) (end 25.55 9.7) (width 0.2) (layer "F.Cu") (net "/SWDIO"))
 (segment (start 23.65 10.75) (end 24.75 9.65) (width 0.2) (layer "F.Cu") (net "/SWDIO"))
 (segment (start 25.55 9.7) (end 25.6 9.7) (width 0.2) (layer "F.Cu") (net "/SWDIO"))
 (segment (start 25.65 9.75) (end 25.7 9.75) (width 0.2) (layer "F.Cu") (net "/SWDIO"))
 (segment (start 25.6 9.7) (end 25.65 9.75) (width 0.2) (layer "F.Cu") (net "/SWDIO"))
 (segment (start 22.65 10.75) (end 23.65 10.75) (width 0.2) (layer "F.Cu") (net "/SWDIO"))
 (segment (start 24.75 9.65) (end 25.5 9.65) (width 0.2) (layer "F.Cu") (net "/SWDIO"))
 (segment (start 26.5 15.35) (end 26.5 15.95) (width 0.2) (layer "F.Cu") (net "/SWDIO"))
 (segment (start 26.6 10.6) (end 26.6 15.25) (width 0.2) (layer "F.Cu") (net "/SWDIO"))
 (segment (start 18.8 16.05) (end 20.35 17.6) (width 0.2) (layer "F.Cu") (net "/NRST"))
 (segment (start 18.15 13.85) (end 18.15 15.4) (width 0.2) (layer "F.Cu") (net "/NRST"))
 (segment (start 18.8 13.2) (end 18.15 13.85) (width 0.2) (layer "F.Cu") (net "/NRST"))
 (segment (start 18.15 15.4) (end 18.8 16.05) (width 0.2) (layer "F.Cu") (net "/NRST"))
 (segment (start 20.35 17.6) (end 21.15 17.6) (width 0.2) (layer "F.Cu") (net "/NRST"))
 (segment (start 21.2 17.65) (end 21.5 17.65) (width 0.2) (layer "F.Cu") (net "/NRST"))
 (segment (start 21.15 17.6) (end 21.2 17.65) (width 0.2) (layer "F.Cu") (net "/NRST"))
 (segment (start 20.1 10.75) (end 18.8 12.05) (width 0.2) (layer "F.Cu") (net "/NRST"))
 (segment (start 18.8 12.05) (end 18.8 13.2) (width 0.2) (layer "F.Cu") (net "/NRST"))
 (segment (start 19.4817 14.6274) (end 20.5243 15.67) (width 0.2) (layer "F.Cu") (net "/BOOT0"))
 (segment (start 21.5 15.67) (end 20.5243 15.67) (width 0.2) (layer "F.Cu") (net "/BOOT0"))
 (segment (start 18.85 14.35) (end 19.4817 14.35) (width 0.2) (layer "F.Cu") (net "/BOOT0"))
 (segment (start 19.4817 14.35) (end 19.4817 14.6274) (width 0.2) (layer "F.Cu") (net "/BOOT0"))
 (segment (start 12.2787 18.92) (end 21.5 18.92) (width 0.2) (layer "F.Cu") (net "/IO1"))
 (segment (start 11.8787 19.32) (end 12.2787 18.92) (width 0.2) (layer "F.Cu") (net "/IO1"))
 (segment (start 10.8 19.32) (end 11.8787 19.32) (width 0.2) (layer "F.Cu") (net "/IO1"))
 (segment (start 13.09 19.57) (end 21.5 19.57) (width 0.2) (layer "F.Cu") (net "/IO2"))
 (segment (start 10.8 21.86) (end 13.09 19.57) (width 0.2) (layer "F.Cu") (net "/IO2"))
 (segment (start 14.98 20.22) (end 21.5 20.22) (width 0.2) (layer "F.Cu") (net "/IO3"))
 (segment (start 10.8 24.4) (end 14.98 20.22) (width 0.2) (layer "F.Cu") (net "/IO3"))
 (segment (start 10.8 26.94) (end 16.87 20.87) (width 0.2) (layer "F.Cu") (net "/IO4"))
 (segment (start 16.87 20.87) (end 21.5 20.87) (width 0.2) (layer "F.Cu") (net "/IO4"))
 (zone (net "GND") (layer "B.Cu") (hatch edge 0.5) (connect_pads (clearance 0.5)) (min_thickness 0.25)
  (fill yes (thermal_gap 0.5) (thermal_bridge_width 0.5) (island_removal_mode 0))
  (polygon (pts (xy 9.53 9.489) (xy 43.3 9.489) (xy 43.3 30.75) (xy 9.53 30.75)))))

